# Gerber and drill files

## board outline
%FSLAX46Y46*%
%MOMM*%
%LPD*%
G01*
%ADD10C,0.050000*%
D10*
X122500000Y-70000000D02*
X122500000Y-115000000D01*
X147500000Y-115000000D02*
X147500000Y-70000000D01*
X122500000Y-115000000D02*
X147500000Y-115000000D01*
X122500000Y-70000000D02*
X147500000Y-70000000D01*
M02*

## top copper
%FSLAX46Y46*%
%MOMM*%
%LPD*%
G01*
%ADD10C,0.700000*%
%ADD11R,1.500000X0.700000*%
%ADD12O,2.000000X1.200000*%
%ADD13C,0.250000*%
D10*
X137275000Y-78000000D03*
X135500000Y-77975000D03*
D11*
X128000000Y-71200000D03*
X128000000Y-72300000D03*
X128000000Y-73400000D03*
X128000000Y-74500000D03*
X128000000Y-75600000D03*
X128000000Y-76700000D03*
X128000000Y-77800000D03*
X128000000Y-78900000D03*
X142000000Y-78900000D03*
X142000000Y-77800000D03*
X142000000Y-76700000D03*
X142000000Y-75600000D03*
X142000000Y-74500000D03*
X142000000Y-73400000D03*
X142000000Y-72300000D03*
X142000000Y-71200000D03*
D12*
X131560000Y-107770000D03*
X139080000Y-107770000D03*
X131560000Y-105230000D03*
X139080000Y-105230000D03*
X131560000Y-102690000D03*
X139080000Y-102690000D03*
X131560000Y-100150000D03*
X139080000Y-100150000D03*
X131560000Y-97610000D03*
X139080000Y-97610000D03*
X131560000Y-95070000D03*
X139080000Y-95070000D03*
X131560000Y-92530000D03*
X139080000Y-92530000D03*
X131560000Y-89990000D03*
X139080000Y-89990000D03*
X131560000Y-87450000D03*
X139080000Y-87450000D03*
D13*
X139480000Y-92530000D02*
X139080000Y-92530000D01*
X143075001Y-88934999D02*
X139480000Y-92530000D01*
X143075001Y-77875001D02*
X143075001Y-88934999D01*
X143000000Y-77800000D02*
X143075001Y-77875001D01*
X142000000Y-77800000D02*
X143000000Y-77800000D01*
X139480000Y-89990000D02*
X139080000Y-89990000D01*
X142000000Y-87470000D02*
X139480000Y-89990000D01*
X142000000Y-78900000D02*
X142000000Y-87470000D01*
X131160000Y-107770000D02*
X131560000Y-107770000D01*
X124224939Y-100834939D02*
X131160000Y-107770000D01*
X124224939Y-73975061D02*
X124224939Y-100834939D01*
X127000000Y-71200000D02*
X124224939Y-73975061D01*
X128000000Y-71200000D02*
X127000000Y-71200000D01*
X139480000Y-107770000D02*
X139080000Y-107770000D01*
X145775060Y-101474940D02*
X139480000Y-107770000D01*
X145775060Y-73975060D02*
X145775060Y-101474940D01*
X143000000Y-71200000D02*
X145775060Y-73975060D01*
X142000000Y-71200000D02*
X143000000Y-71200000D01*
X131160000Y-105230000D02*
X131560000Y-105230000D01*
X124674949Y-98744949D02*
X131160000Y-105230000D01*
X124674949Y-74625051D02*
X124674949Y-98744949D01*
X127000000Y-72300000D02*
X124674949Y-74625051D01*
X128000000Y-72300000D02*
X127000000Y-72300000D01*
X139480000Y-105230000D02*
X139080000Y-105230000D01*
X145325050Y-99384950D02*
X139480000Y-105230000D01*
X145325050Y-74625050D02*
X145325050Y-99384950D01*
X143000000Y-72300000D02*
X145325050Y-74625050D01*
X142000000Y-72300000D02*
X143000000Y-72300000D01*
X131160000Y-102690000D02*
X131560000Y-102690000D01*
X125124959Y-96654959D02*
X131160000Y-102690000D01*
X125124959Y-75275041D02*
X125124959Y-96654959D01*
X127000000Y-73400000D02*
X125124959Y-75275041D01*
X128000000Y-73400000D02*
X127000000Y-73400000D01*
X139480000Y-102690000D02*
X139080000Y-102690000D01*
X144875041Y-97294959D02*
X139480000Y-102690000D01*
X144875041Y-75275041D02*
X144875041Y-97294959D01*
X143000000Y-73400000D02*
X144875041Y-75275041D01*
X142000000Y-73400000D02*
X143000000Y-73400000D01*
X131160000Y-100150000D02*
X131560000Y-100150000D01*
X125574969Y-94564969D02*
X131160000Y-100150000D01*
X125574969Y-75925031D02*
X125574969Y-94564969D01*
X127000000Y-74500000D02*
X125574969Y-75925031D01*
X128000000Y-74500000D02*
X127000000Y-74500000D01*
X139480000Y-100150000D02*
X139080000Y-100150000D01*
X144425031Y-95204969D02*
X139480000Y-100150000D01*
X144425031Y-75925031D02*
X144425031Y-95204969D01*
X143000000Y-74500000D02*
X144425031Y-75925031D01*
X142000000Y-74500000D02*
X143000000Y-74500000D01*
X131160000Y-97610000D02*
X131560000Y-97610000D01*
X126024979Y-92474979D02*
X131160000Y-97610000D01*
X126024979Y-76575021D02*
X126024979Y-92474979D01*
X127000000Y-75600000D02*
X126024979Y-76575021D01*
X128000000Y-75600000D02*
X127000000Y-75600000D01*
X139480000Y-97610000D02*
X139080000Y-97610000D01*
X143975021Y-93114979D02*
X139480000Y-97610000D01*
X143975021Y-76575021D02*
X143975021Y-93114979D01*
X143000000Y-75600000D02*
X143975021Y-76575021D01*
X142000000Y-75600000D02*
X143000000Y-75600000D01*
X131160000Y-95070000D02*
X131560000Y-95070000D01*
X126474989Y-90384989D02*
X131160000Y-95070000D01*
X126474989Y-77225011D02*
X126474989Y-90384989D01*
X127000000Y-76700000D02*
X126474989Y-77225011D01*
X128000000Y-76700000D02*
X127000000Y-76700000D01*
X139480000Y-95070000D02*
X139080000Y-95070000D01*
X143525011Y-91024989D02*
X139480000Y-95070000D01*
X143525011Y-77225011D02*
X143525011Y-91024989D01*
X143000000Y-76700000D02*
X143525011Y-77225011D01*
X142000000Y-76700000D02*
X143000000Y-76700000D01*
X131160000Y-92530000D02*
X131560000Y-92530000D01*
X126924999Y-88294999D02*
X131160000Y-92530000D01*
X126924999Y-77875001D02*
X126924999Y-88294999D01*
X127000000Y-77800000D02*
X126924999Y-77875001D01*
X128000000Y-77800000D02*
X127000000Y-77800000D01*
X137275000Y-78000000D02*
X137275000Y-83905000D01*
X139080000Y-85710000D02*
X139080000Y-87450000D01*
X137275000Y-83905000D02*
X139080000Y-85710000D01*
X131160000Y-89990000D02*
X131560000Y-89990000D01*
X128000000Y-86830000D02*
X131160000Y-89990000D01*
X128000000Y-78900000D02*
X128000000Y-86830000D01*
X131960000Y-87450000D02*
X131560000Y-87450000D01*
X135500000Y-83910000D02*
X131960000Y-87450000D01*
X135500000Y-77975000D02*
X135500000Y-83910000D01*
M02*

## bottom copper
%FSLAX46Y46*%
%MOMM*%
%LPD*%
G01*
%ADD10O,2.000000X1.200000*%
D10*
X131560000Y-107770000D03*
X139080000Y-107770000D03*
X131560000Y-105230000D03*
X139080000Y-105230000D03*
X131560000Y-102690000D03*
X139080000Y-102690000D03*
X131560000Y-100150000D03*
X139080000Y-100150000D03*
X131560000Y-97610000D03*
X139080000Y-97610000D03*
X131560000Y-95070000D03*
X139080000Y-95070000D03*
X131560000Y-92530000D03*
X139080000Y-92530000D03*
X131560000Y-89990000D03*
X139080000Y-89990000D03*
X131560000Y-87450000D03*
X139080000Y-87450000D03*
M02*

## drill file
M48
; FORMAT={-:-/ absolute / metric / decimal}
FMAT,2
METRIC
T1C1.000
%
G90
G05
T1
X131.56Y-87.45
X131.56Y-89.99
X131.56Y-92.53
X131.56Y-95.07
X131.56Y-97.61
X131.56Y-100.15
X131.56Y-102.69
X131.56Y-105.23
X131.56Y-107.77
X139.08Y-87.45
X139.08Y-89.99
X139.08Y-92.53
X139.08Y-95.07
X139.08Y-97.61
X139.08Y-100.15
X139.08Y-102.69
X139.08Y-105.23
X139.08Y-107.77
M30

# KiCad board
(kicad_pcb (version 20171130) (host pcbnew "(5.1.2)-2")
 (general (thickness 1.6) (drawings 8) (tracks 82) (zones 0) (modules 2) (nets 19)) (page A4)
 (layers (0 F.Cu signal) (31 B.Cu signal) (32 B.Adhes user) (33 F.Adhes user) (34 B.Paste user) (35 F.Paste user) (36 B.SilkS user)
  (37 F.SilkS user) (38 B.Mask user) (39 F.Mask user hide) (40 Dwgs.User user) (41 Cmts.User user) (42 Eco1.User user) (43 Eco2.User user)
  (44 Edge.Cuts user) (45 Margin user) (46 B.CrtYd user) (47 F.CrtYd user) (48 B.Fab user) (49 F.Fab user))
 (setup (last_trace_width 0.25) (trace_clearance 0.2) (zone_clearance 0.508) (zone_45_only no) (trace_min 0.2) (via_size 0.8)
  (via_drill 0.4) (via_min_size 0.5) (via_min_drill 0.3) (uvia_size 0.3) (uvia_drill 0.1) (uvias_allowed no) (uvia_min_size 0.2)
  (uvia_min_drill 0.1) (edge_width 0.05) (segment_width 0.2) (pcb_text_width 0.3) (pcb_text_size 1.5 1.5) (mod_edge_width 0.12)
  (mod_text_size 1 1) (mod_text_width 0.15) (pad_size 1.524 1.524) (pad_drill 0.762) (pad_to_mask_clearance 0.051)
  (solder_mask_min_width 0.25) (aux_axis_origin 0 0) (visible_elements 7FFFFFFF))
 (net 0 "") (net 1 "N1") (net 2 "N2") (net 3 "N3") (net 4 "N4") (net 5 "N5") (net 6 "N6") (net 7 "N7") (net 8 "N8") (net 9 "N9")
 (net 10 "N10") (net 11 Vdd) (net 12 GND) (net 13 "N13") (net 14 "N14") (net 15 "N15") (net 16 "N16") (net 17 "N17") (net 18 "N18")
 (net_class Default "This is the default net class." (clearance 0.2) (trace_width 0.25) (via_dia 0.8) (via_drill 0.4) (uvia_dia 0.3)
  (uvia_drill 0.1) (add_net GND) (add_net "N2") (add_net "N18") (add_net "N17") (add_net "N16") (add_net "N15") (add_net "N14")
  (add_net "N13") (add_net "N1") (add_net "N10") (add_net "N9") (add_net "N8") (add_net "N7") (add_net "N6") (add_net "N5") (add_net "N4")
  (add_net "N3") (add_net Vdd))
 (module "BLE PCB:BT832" (layer F.Cu) (at 135 72)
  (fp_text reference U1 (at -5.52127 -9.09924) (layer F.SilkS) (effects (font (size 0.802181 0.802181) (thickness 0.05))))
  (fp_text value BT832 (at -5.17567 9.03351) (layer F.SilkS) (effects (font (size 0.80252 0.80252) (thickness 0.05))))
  (pad D5 smd circle (at 2.275 6) (size 0.7 0.7) (layers F.Cu F.Paste F.Mask) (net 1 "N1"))
  (pad C5 smd circle (at 0.5 5.975) (size 0.7 0.7) (layers F.Cu F.Paste F.Mask) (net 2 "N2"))
  (pad 1 smd rect (at -7 -0.8) (size 1.5 0.7) (layers F.Cu F.Paste F.Mask) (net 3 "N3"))
  (pad 2 smd rect (at -7 0.3) (size 1.5 0.7) (layers F.Cu F.Paste F.Mask) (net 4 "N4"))
  (pad 3 smd rect (at -7 1.4) (size 1.5 0.7) (layers F.Cu F.Paste F.Mask) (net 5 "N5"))
  (pad 4 smd rect (at -7 2.5) (size 1.5 0.7) (layers F.Cu F.Paste F.Mask) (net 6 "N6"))
  (pad 5 smd rect (at -7 3.6) (size 1.5 0.7) (layers F.Cu F.Paste F.Mask) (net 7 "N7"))
  (pad 6 smd rect (at -7 4.7) (size 1.5 0.7) (layers F.Cu F.Paste F.Mask) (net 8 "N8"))
  (pad 7 smd rect (at -7 5.8) (size 1.5 0.7) (layers F.Cu F.Paste F.Mask) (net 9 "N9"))
  (pad 8 smd rect (at -7 6.9) (size 1.5 0.7) (layers F.Cu F.Paste F.Mask) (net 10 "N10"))
  (pad 9 smd rect (at 7 6.9 180) (size 1.5 0.7) (layers F.Cu F.Paste F.Mask) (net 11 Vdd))
  (pad 10 smd rect (at 7 5.8 180) (size 1.5 0.7) (layers F.Cu F.Paste F.Mask) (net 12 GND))
  (pad 11 smd rect (at 7 4.7 180) (size 1.5 0.7) (layers F.Cu F.Paste F.Mask) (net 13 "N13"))
  (pad 12 smd rect (at 7 3.6 180) (size 1.5 0.7) (layers F.Cu F.Paste F.Mask) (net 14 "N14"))
  (pad 13 smd rect (at 7 2.5 180) (size 1.5 0.7) (layers F.Cu F.Paste F.Mask) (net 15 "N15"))
  (pad 14 smd rect (at 7 1.4 180) (size 1.5 0.7) (layers F.Cu F.Paste F.Mask) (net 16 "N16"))
  (pad 15 smd rect (at 7 0.3 180) (size 1.5 0.7) (layers F.Cu F.Paste F.Mask) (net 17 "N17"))
  (pad 16 smd rect (at 7 -0.8 180) (size 1.5 0.7) (layers F.Cu F.Paste F.Mask) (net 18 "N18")))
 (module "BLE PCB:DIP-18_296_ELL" (layer F.Cu) (at 135.32 97.61 270)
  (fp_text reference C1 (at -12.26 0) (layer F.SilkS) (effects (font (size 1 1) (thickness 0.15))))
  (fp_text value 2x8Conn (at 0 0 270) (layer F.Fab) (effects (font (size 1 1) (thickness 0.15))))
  (pad 9 thru_hole oval (at 10.16 3.76 270) (size 1.2 2) (drill 1) (layers *.Cu *.Mask) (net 3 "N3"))
  (pad 10 thru_hole oval (at 10.16 -3.76 270) (size 1.2 2) (drill 1) (layers *.Cu *.Mask) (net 18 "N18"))
  (pad 8 thru_hole oval (at 7.62 3.76 270) (size 1.2 2) (drill 1) (layers *.Cu *.Mask) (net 4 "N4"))
  (pad 11 thru_hole oval (at 7.62 -3.76 270) (size 1.2 2) (drill 1) (layers *.Cu *.Mask) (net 17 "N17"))
  (pad 7 thru_hole oval (at 5.08 3.76 270) (size 1.2 2) (drill 1) (layers *.Cu *.Mask) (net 5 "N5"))
  (pad 12 thru_hole oval (at 5.08 -3.76 270) (size 1.2 2) (drill 1) (layers *.Cu *.Mask) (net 16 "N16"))
  (pad 6 thru_hole oval (at 2.54 3.76 270) (size 1.2 2) (drill 1) (layers *.Cu *.Mask) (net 6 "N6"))
  (pad 13 thru_hole oval (at 2.54 -3.76 270) (size 1.2 2) (drill 1) (layers *.Cu *.Mask) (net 15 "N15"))
  (pad 5 thru_hole oval (at 0 3.76 270) (size 1.2 2) (drill 1) (layers *.Cu *.Mask) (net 7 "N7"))
  (pad 14 thru_hole oval (at 0 -3.76 270) (size 1.2 2) (drill 1) (layers *.Cu *.Mask) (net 14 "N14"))
  (pad 4 thru_hole oval (at -2.54 3.76 270) (size 1.2 2) (drill 1) (layers *.Cu *.Mask) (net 8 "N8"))
  (pad 15 thru_hole oval (at -2.54 -3.76 270) (size 1.2 2) (drill 1) (layers *.Cu *.Mask) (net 13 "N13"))
  (pad 3 thru_hole oval (at -5.08 3.76 270) (size 1.2 2) (drill 1) (layers *.Cu *.Mask) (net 9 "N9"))
  (pad 16 thru_hole oval (at -5.08 -3.76 270) (size 1.2 2) (drill 1) (layers *.Cu *.Mask) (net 12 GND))
  (pad 2 thru_hole oval (at -7.62 3.76 270) (size 1.2 2) (drill 1) (layers *.Cu *.Mask) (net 10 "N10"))
  (pad 17 thru_hole oval (at -7.62 -3.76 270) (size 1.2 2) (drill 1) (layers *.Cu *.Mask) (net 11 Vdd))
  (pad 1 thru_hole oval (at -10.16 3.76 270) (size 1.2 2) (drill 1) (layers *.Cu *.Mask) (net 2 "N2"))
  (pad 18 thru_hole oval (at -10.16 -3.76 270) (size 1.2 2) (drill 1) (layers *.Cu *.Mask) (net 1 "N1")))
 (gr_line (start 122.5 70) (end 122.5 115) (layer Edge.Cuts) (width 0.05))
 (gr_line (start 147.5 115) (end 147.5 70) (layer Edge.Cuts) (width 0.05))
 (gr_line (start 122.5 115) (end 147.5 115) (layer Edge.Cuts) (width 0.05))
 (gr_line (start 122.5 70) (end 147.5 70) (layer Edge.Cuts) (width 0.05))
 (segment (start 139.48 92.53) (end 139.08 92.53) (width 0.25) (layer F.Cu) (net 12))
 (segment (start 143.075001 88.934999) (end 139.48 92.53) (width 0.25) (layer F.Cu) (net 12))
 (segment (start 143.075001 77.875001) (end 143.075001 88.934999) (width 0.25) (layer F.Cu) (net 12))
 (segment (start 143 77.8) (end 143.075001 77.875001) (width 0.25) (layer F.Cu) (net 12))
 (segment (start 142 77.8) (end 143 77.8) (width 0.25) (layer F.Cu) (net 12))
 (segment (start 139.48 89.99) (end 139.08 89.99) (width 0.25) (layer F.Cu) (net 11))
 (segment (start 142 87.47) (end 139.48 89.99) (width 0.25) (layer F.Cu) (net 11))
 (segment (start 142 78.9) (end 142 87.47) (width 0.25) (layer F.Cu) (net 11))
 (segment (start 131.16 107.77) (end 131.56 107.77) (width 0.25) (layer F.Cu) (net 3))
 (segment (start 124.224939 100.834939) (end 131.16 107.77) (width 0.25) (layer F.Cu) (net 3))
 (segment (start 124.224939 73.975061) (end 124.224939 100.834939) (width 0.25) (layer F.Cu) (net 3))
 (segment (start 127 71.2) (end 124.224939 73.975061) (width 0.25) (layer F.Cu) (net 3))
 (segment (start 128 71.2) (end 127 71.2) (width 0.25) (layer F.Cu) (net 3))
 (segment (start 139.48 107.77) (end 139.08 107.77) (width 0.25) (layer F.Cu) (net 18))
 (segment (start 145.77506 101.47494) (end 139.48 107.77) (width 0.25) (layer F.Cu) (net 18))
 (segment (start 145.77506 73.97506) (end 145.77506 101.47494) (width 0.25) (layer F.Cu) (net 18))
 (segment (start 143 71.2) (end 145.77506 73.97506) (width 0.25) (layer F.Cu) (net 18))
 (segment (start 142 71.2) (end 143 71.2) (width 0.25) (layer F.Cu) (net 18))
 (segment (start 131.16 105.23) (end 131.56 105.23) (width 0.25) (layer F.Cu) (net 4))
 (segment (start 124.674949 98.744949) (end 131.16 105.23) (width 0.25) (layer F.Cu) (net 4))
 (segment (start 124.674949 74.625051) (end 124.674949 98.744949) (width 0.25) (layer F.Cu) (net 4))
 (segment (start 127 72.3) (end 124.674949 74.625051) (width 0.25) (layer F.Cu) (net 4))
 (segment (start 128 72.3) (end 127 72.3) (width 0.25) (layer F.Cu) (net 4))
 (segment (start 139.48 105.23) (end 139.08 105.23) (width 0.25) (layer F.Cu) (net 17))
 (segment (start 145.32505 99.38495) (end 139.48 105.23) (width 0.25) (layer F.Cu) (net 17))
 (segment (start 145.32505 74.62505) (end 145.32505 99.38495) (width 0.25) (layer F.Cu) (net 17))
 (segment (start 143 72.3) (end 145.32505 74.62505) (width 0.25) (layer F.Cu) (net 17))
 (segment (start 142 72.3) (end 143 72.3) (width 0.25) (layer F.Cu) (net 17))
 (segment (start 131.16 102.69) (end 131.56 102.69) (width 0.25) (layer F.Cu) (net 5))
 (segment (start 125.124959 96.654959) (end 131.16 102.69) (width 0.25) (layer F.Cu) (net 5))
 (segment (start 125.124959 75.275041) (end 125.124959 96.654959) (width 0.25) (layer F.Cu) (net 5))
 (segment (start 127 73.4) (end 125.124959 75.275041) (width 0.25) (layer F.Cu) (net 5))
 (segment (start 128 73.4) (end 127 73.4) (width 0.25) (layer F.Cu) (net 5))
 (segment (start 139.48 102.69) (end 139.08 102.69) (width 0.25) (layer F.Cu) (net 16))
 (segment (start 144.875041 97.294959) (end 139.48 102.69) (width 0.25) (layer F.Cu) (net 16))
 (segment (start 144.875041 75.275041) (end 144.875041 97.294959) (width 0.25) (layer F.Cu) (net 16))
 (segment (start 143 73.4) (end 144.875041 75.275041) (width 0.25) (layer F.Cu) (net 16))
 (segment (start 142 73.4) (end 143 73.4) (width 0.25) (layer F.Cu) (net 16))
 (segment (start 131.16 100.15) (end 131.56 100.15) (width 0.25) (layer F.Cu) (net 6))
 (segment (start 125.574969 94.564969) (end 131.16 100.15) (width 0.25) (layer F.Cu) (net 6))
 (segment (start 125.574969 75.925031) (end 125.574969 94.564969) (width 0.25) (layer F.Cu) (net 6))
 (segment (start 127 74.5) (end 125.574969 75.925031) (width 0.25) (layer F.Cu) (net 6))
 (segment (start 128 74.5) (end 127 74.5) (width 0.25) (layer F.Cu) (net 6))
 (segment (start 139.48 100.15) (end 139.08 100.15) (width 0.25) (layer F.Cu) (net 15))
 (segment (start 144.425031 95.204969) (end 139.48 100.15) (width 0.25) (layer F.Cu) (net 15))
 (segment (start 144.425031 75.925031) (end 144.425031 95.204969) (width 0.25) (layer F.Cu) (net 15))
 (segment (start 143 74.5) (end 144.425031 75.925031) (width 0.25) (layer F.Cu) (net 15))
 (segment (start 142 74.5) (end 143 74.5) (width 0.25) (layer F.Cu) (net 15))
 (segment (start 131.16 97.61) (end 131.56 97.61) (width 0.25) (layer F.Cu) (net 7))
 (segment (start 126.024979 92.474979) (end 131.16 97.61) (width 0.25) (layer F.Cu) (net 7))
 (segment (start 126.024979 76.575021) (end 126.024979 92.474979) (width 0.25) (layer F.Cu) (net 7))
 (segment (start 127 75.6) (end 126.024979 76.575021) (width 0.25) (layer F.Cu) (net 7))
 (segment (start 128 75.6) (end 127 75.6) (width 0.25) (layer F.Cu) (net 7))
 (segment (start 139.48 97.61) (end 139.08 97.61) (width 0.25) (layer F.Cu) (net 14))
 (segment (start 143.975021 93.114979) (end 139.48 97.61) (width 0.25) (layer F.Cu) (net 14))
 (segment (start 143.975021 76.575021) (end 143.975021 93.114979) (width 0.25) (layer F.Cu) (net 14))
 (segment (start 143 75.6) (end 143.975021 76.575021) (width 0.25) (layer F.Cu) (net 14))
 (segment (start 142 75.6) (end 143 75.6) (width 0.25) (layer F.Cu) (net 14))
 (segment (start 131.16 95.07) (end 131.56 95.07) (width 0.25) (layer F.Cu) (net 8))
 (segment (start 126.474989 90.384989) (end 131.16 95.07) (width 0.25) (layer F.Cu) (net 8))
 (segment (start 126.474989 77.225011) (end 126.474989 90.384989) (width 0.25) (layer F.Cu) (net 8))
 (segment (start 127 76.7) (end 126.474989 77.225011) (width 0.25) (layer F.Cu) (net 8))
 (segment (start 128 76.7) (end 127 76.7) (width 0.25) (layer F.Cu) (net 8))
 (segment (start 139.48 95.07) (end 139.08 95.07) (width 0.25) (layer F.Cu) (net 13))
 (segment (start 143.525011 91.024989) (end 139.48 95.07) (width 0.25) (layer F.Cu) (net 13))
 (segment (start 143.525011 77.225011) (end 143.525011 91.024989) (width 0.25) (layer F.Cu) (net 13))
 (segment (start 143 76.7) (end 143.525011 77.225011) (width 0.25) (layer F.Cu) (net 13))
 (segment (start 142 76.7) (end 143 76.7) (width 0.25) (layer F.Cu) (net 13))
 (segment (start 131.16 92.53) (end 131.56 92.53) (width 0.25) (layer F.Cu) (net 9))
 (segment (start 126.924999 88.294999) (end 131.16 92.53) (width 0.25) (layer F.Cu) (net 9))
 (segment (start 126.924999 77.875001) (end 126.924999 88.294999) (width 0.25) (layer F.Cu) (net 9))
 (segment (start 127 77.8) (end 126.924999 77.875001) (width 0.25) (layer F.Cu) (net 9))
 (segment (start 128 77.8) (end 127 77.8) (width 0.25) (layer F.Cu) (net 9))
 (segment (start 137.275 78) (end 137.275 83.905) (width 0.25) (layer F.Cu) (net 1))
 (segment (start 139.08 85.71) (end 139.08 87.45) (width 0.25) (layer F.Cu) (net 1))
 (segment (start 137.275 83.905) (end 139.08 85.71) (width 0.25) (layer F.Cu) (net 1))
 (segment (start 131.16 89.99) (end 131.56 89.99) (width 0.25) (layer F.Cu) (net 10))
 (segment (start 128 86.83) (end 131.16 89.99) (width 0.25) (layer F.Cu) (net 10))
 (segment (start 128 78.9) (end 128 86.83) (width 0.25) (layer F.Cu) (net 10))
 (segment (start 131.96 87.45) (end 131.56 87.45) (width 0.25) (layer F.Cu) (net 2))
 (segment (start 135.5 83.91) (end 131.96 87.45) (width 0.25) (layer F.Cu) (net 2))
 (segment (start 135.5 77.975) (end 135.5 83.91) (width 0.25) (layer F.Cu) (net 2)))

